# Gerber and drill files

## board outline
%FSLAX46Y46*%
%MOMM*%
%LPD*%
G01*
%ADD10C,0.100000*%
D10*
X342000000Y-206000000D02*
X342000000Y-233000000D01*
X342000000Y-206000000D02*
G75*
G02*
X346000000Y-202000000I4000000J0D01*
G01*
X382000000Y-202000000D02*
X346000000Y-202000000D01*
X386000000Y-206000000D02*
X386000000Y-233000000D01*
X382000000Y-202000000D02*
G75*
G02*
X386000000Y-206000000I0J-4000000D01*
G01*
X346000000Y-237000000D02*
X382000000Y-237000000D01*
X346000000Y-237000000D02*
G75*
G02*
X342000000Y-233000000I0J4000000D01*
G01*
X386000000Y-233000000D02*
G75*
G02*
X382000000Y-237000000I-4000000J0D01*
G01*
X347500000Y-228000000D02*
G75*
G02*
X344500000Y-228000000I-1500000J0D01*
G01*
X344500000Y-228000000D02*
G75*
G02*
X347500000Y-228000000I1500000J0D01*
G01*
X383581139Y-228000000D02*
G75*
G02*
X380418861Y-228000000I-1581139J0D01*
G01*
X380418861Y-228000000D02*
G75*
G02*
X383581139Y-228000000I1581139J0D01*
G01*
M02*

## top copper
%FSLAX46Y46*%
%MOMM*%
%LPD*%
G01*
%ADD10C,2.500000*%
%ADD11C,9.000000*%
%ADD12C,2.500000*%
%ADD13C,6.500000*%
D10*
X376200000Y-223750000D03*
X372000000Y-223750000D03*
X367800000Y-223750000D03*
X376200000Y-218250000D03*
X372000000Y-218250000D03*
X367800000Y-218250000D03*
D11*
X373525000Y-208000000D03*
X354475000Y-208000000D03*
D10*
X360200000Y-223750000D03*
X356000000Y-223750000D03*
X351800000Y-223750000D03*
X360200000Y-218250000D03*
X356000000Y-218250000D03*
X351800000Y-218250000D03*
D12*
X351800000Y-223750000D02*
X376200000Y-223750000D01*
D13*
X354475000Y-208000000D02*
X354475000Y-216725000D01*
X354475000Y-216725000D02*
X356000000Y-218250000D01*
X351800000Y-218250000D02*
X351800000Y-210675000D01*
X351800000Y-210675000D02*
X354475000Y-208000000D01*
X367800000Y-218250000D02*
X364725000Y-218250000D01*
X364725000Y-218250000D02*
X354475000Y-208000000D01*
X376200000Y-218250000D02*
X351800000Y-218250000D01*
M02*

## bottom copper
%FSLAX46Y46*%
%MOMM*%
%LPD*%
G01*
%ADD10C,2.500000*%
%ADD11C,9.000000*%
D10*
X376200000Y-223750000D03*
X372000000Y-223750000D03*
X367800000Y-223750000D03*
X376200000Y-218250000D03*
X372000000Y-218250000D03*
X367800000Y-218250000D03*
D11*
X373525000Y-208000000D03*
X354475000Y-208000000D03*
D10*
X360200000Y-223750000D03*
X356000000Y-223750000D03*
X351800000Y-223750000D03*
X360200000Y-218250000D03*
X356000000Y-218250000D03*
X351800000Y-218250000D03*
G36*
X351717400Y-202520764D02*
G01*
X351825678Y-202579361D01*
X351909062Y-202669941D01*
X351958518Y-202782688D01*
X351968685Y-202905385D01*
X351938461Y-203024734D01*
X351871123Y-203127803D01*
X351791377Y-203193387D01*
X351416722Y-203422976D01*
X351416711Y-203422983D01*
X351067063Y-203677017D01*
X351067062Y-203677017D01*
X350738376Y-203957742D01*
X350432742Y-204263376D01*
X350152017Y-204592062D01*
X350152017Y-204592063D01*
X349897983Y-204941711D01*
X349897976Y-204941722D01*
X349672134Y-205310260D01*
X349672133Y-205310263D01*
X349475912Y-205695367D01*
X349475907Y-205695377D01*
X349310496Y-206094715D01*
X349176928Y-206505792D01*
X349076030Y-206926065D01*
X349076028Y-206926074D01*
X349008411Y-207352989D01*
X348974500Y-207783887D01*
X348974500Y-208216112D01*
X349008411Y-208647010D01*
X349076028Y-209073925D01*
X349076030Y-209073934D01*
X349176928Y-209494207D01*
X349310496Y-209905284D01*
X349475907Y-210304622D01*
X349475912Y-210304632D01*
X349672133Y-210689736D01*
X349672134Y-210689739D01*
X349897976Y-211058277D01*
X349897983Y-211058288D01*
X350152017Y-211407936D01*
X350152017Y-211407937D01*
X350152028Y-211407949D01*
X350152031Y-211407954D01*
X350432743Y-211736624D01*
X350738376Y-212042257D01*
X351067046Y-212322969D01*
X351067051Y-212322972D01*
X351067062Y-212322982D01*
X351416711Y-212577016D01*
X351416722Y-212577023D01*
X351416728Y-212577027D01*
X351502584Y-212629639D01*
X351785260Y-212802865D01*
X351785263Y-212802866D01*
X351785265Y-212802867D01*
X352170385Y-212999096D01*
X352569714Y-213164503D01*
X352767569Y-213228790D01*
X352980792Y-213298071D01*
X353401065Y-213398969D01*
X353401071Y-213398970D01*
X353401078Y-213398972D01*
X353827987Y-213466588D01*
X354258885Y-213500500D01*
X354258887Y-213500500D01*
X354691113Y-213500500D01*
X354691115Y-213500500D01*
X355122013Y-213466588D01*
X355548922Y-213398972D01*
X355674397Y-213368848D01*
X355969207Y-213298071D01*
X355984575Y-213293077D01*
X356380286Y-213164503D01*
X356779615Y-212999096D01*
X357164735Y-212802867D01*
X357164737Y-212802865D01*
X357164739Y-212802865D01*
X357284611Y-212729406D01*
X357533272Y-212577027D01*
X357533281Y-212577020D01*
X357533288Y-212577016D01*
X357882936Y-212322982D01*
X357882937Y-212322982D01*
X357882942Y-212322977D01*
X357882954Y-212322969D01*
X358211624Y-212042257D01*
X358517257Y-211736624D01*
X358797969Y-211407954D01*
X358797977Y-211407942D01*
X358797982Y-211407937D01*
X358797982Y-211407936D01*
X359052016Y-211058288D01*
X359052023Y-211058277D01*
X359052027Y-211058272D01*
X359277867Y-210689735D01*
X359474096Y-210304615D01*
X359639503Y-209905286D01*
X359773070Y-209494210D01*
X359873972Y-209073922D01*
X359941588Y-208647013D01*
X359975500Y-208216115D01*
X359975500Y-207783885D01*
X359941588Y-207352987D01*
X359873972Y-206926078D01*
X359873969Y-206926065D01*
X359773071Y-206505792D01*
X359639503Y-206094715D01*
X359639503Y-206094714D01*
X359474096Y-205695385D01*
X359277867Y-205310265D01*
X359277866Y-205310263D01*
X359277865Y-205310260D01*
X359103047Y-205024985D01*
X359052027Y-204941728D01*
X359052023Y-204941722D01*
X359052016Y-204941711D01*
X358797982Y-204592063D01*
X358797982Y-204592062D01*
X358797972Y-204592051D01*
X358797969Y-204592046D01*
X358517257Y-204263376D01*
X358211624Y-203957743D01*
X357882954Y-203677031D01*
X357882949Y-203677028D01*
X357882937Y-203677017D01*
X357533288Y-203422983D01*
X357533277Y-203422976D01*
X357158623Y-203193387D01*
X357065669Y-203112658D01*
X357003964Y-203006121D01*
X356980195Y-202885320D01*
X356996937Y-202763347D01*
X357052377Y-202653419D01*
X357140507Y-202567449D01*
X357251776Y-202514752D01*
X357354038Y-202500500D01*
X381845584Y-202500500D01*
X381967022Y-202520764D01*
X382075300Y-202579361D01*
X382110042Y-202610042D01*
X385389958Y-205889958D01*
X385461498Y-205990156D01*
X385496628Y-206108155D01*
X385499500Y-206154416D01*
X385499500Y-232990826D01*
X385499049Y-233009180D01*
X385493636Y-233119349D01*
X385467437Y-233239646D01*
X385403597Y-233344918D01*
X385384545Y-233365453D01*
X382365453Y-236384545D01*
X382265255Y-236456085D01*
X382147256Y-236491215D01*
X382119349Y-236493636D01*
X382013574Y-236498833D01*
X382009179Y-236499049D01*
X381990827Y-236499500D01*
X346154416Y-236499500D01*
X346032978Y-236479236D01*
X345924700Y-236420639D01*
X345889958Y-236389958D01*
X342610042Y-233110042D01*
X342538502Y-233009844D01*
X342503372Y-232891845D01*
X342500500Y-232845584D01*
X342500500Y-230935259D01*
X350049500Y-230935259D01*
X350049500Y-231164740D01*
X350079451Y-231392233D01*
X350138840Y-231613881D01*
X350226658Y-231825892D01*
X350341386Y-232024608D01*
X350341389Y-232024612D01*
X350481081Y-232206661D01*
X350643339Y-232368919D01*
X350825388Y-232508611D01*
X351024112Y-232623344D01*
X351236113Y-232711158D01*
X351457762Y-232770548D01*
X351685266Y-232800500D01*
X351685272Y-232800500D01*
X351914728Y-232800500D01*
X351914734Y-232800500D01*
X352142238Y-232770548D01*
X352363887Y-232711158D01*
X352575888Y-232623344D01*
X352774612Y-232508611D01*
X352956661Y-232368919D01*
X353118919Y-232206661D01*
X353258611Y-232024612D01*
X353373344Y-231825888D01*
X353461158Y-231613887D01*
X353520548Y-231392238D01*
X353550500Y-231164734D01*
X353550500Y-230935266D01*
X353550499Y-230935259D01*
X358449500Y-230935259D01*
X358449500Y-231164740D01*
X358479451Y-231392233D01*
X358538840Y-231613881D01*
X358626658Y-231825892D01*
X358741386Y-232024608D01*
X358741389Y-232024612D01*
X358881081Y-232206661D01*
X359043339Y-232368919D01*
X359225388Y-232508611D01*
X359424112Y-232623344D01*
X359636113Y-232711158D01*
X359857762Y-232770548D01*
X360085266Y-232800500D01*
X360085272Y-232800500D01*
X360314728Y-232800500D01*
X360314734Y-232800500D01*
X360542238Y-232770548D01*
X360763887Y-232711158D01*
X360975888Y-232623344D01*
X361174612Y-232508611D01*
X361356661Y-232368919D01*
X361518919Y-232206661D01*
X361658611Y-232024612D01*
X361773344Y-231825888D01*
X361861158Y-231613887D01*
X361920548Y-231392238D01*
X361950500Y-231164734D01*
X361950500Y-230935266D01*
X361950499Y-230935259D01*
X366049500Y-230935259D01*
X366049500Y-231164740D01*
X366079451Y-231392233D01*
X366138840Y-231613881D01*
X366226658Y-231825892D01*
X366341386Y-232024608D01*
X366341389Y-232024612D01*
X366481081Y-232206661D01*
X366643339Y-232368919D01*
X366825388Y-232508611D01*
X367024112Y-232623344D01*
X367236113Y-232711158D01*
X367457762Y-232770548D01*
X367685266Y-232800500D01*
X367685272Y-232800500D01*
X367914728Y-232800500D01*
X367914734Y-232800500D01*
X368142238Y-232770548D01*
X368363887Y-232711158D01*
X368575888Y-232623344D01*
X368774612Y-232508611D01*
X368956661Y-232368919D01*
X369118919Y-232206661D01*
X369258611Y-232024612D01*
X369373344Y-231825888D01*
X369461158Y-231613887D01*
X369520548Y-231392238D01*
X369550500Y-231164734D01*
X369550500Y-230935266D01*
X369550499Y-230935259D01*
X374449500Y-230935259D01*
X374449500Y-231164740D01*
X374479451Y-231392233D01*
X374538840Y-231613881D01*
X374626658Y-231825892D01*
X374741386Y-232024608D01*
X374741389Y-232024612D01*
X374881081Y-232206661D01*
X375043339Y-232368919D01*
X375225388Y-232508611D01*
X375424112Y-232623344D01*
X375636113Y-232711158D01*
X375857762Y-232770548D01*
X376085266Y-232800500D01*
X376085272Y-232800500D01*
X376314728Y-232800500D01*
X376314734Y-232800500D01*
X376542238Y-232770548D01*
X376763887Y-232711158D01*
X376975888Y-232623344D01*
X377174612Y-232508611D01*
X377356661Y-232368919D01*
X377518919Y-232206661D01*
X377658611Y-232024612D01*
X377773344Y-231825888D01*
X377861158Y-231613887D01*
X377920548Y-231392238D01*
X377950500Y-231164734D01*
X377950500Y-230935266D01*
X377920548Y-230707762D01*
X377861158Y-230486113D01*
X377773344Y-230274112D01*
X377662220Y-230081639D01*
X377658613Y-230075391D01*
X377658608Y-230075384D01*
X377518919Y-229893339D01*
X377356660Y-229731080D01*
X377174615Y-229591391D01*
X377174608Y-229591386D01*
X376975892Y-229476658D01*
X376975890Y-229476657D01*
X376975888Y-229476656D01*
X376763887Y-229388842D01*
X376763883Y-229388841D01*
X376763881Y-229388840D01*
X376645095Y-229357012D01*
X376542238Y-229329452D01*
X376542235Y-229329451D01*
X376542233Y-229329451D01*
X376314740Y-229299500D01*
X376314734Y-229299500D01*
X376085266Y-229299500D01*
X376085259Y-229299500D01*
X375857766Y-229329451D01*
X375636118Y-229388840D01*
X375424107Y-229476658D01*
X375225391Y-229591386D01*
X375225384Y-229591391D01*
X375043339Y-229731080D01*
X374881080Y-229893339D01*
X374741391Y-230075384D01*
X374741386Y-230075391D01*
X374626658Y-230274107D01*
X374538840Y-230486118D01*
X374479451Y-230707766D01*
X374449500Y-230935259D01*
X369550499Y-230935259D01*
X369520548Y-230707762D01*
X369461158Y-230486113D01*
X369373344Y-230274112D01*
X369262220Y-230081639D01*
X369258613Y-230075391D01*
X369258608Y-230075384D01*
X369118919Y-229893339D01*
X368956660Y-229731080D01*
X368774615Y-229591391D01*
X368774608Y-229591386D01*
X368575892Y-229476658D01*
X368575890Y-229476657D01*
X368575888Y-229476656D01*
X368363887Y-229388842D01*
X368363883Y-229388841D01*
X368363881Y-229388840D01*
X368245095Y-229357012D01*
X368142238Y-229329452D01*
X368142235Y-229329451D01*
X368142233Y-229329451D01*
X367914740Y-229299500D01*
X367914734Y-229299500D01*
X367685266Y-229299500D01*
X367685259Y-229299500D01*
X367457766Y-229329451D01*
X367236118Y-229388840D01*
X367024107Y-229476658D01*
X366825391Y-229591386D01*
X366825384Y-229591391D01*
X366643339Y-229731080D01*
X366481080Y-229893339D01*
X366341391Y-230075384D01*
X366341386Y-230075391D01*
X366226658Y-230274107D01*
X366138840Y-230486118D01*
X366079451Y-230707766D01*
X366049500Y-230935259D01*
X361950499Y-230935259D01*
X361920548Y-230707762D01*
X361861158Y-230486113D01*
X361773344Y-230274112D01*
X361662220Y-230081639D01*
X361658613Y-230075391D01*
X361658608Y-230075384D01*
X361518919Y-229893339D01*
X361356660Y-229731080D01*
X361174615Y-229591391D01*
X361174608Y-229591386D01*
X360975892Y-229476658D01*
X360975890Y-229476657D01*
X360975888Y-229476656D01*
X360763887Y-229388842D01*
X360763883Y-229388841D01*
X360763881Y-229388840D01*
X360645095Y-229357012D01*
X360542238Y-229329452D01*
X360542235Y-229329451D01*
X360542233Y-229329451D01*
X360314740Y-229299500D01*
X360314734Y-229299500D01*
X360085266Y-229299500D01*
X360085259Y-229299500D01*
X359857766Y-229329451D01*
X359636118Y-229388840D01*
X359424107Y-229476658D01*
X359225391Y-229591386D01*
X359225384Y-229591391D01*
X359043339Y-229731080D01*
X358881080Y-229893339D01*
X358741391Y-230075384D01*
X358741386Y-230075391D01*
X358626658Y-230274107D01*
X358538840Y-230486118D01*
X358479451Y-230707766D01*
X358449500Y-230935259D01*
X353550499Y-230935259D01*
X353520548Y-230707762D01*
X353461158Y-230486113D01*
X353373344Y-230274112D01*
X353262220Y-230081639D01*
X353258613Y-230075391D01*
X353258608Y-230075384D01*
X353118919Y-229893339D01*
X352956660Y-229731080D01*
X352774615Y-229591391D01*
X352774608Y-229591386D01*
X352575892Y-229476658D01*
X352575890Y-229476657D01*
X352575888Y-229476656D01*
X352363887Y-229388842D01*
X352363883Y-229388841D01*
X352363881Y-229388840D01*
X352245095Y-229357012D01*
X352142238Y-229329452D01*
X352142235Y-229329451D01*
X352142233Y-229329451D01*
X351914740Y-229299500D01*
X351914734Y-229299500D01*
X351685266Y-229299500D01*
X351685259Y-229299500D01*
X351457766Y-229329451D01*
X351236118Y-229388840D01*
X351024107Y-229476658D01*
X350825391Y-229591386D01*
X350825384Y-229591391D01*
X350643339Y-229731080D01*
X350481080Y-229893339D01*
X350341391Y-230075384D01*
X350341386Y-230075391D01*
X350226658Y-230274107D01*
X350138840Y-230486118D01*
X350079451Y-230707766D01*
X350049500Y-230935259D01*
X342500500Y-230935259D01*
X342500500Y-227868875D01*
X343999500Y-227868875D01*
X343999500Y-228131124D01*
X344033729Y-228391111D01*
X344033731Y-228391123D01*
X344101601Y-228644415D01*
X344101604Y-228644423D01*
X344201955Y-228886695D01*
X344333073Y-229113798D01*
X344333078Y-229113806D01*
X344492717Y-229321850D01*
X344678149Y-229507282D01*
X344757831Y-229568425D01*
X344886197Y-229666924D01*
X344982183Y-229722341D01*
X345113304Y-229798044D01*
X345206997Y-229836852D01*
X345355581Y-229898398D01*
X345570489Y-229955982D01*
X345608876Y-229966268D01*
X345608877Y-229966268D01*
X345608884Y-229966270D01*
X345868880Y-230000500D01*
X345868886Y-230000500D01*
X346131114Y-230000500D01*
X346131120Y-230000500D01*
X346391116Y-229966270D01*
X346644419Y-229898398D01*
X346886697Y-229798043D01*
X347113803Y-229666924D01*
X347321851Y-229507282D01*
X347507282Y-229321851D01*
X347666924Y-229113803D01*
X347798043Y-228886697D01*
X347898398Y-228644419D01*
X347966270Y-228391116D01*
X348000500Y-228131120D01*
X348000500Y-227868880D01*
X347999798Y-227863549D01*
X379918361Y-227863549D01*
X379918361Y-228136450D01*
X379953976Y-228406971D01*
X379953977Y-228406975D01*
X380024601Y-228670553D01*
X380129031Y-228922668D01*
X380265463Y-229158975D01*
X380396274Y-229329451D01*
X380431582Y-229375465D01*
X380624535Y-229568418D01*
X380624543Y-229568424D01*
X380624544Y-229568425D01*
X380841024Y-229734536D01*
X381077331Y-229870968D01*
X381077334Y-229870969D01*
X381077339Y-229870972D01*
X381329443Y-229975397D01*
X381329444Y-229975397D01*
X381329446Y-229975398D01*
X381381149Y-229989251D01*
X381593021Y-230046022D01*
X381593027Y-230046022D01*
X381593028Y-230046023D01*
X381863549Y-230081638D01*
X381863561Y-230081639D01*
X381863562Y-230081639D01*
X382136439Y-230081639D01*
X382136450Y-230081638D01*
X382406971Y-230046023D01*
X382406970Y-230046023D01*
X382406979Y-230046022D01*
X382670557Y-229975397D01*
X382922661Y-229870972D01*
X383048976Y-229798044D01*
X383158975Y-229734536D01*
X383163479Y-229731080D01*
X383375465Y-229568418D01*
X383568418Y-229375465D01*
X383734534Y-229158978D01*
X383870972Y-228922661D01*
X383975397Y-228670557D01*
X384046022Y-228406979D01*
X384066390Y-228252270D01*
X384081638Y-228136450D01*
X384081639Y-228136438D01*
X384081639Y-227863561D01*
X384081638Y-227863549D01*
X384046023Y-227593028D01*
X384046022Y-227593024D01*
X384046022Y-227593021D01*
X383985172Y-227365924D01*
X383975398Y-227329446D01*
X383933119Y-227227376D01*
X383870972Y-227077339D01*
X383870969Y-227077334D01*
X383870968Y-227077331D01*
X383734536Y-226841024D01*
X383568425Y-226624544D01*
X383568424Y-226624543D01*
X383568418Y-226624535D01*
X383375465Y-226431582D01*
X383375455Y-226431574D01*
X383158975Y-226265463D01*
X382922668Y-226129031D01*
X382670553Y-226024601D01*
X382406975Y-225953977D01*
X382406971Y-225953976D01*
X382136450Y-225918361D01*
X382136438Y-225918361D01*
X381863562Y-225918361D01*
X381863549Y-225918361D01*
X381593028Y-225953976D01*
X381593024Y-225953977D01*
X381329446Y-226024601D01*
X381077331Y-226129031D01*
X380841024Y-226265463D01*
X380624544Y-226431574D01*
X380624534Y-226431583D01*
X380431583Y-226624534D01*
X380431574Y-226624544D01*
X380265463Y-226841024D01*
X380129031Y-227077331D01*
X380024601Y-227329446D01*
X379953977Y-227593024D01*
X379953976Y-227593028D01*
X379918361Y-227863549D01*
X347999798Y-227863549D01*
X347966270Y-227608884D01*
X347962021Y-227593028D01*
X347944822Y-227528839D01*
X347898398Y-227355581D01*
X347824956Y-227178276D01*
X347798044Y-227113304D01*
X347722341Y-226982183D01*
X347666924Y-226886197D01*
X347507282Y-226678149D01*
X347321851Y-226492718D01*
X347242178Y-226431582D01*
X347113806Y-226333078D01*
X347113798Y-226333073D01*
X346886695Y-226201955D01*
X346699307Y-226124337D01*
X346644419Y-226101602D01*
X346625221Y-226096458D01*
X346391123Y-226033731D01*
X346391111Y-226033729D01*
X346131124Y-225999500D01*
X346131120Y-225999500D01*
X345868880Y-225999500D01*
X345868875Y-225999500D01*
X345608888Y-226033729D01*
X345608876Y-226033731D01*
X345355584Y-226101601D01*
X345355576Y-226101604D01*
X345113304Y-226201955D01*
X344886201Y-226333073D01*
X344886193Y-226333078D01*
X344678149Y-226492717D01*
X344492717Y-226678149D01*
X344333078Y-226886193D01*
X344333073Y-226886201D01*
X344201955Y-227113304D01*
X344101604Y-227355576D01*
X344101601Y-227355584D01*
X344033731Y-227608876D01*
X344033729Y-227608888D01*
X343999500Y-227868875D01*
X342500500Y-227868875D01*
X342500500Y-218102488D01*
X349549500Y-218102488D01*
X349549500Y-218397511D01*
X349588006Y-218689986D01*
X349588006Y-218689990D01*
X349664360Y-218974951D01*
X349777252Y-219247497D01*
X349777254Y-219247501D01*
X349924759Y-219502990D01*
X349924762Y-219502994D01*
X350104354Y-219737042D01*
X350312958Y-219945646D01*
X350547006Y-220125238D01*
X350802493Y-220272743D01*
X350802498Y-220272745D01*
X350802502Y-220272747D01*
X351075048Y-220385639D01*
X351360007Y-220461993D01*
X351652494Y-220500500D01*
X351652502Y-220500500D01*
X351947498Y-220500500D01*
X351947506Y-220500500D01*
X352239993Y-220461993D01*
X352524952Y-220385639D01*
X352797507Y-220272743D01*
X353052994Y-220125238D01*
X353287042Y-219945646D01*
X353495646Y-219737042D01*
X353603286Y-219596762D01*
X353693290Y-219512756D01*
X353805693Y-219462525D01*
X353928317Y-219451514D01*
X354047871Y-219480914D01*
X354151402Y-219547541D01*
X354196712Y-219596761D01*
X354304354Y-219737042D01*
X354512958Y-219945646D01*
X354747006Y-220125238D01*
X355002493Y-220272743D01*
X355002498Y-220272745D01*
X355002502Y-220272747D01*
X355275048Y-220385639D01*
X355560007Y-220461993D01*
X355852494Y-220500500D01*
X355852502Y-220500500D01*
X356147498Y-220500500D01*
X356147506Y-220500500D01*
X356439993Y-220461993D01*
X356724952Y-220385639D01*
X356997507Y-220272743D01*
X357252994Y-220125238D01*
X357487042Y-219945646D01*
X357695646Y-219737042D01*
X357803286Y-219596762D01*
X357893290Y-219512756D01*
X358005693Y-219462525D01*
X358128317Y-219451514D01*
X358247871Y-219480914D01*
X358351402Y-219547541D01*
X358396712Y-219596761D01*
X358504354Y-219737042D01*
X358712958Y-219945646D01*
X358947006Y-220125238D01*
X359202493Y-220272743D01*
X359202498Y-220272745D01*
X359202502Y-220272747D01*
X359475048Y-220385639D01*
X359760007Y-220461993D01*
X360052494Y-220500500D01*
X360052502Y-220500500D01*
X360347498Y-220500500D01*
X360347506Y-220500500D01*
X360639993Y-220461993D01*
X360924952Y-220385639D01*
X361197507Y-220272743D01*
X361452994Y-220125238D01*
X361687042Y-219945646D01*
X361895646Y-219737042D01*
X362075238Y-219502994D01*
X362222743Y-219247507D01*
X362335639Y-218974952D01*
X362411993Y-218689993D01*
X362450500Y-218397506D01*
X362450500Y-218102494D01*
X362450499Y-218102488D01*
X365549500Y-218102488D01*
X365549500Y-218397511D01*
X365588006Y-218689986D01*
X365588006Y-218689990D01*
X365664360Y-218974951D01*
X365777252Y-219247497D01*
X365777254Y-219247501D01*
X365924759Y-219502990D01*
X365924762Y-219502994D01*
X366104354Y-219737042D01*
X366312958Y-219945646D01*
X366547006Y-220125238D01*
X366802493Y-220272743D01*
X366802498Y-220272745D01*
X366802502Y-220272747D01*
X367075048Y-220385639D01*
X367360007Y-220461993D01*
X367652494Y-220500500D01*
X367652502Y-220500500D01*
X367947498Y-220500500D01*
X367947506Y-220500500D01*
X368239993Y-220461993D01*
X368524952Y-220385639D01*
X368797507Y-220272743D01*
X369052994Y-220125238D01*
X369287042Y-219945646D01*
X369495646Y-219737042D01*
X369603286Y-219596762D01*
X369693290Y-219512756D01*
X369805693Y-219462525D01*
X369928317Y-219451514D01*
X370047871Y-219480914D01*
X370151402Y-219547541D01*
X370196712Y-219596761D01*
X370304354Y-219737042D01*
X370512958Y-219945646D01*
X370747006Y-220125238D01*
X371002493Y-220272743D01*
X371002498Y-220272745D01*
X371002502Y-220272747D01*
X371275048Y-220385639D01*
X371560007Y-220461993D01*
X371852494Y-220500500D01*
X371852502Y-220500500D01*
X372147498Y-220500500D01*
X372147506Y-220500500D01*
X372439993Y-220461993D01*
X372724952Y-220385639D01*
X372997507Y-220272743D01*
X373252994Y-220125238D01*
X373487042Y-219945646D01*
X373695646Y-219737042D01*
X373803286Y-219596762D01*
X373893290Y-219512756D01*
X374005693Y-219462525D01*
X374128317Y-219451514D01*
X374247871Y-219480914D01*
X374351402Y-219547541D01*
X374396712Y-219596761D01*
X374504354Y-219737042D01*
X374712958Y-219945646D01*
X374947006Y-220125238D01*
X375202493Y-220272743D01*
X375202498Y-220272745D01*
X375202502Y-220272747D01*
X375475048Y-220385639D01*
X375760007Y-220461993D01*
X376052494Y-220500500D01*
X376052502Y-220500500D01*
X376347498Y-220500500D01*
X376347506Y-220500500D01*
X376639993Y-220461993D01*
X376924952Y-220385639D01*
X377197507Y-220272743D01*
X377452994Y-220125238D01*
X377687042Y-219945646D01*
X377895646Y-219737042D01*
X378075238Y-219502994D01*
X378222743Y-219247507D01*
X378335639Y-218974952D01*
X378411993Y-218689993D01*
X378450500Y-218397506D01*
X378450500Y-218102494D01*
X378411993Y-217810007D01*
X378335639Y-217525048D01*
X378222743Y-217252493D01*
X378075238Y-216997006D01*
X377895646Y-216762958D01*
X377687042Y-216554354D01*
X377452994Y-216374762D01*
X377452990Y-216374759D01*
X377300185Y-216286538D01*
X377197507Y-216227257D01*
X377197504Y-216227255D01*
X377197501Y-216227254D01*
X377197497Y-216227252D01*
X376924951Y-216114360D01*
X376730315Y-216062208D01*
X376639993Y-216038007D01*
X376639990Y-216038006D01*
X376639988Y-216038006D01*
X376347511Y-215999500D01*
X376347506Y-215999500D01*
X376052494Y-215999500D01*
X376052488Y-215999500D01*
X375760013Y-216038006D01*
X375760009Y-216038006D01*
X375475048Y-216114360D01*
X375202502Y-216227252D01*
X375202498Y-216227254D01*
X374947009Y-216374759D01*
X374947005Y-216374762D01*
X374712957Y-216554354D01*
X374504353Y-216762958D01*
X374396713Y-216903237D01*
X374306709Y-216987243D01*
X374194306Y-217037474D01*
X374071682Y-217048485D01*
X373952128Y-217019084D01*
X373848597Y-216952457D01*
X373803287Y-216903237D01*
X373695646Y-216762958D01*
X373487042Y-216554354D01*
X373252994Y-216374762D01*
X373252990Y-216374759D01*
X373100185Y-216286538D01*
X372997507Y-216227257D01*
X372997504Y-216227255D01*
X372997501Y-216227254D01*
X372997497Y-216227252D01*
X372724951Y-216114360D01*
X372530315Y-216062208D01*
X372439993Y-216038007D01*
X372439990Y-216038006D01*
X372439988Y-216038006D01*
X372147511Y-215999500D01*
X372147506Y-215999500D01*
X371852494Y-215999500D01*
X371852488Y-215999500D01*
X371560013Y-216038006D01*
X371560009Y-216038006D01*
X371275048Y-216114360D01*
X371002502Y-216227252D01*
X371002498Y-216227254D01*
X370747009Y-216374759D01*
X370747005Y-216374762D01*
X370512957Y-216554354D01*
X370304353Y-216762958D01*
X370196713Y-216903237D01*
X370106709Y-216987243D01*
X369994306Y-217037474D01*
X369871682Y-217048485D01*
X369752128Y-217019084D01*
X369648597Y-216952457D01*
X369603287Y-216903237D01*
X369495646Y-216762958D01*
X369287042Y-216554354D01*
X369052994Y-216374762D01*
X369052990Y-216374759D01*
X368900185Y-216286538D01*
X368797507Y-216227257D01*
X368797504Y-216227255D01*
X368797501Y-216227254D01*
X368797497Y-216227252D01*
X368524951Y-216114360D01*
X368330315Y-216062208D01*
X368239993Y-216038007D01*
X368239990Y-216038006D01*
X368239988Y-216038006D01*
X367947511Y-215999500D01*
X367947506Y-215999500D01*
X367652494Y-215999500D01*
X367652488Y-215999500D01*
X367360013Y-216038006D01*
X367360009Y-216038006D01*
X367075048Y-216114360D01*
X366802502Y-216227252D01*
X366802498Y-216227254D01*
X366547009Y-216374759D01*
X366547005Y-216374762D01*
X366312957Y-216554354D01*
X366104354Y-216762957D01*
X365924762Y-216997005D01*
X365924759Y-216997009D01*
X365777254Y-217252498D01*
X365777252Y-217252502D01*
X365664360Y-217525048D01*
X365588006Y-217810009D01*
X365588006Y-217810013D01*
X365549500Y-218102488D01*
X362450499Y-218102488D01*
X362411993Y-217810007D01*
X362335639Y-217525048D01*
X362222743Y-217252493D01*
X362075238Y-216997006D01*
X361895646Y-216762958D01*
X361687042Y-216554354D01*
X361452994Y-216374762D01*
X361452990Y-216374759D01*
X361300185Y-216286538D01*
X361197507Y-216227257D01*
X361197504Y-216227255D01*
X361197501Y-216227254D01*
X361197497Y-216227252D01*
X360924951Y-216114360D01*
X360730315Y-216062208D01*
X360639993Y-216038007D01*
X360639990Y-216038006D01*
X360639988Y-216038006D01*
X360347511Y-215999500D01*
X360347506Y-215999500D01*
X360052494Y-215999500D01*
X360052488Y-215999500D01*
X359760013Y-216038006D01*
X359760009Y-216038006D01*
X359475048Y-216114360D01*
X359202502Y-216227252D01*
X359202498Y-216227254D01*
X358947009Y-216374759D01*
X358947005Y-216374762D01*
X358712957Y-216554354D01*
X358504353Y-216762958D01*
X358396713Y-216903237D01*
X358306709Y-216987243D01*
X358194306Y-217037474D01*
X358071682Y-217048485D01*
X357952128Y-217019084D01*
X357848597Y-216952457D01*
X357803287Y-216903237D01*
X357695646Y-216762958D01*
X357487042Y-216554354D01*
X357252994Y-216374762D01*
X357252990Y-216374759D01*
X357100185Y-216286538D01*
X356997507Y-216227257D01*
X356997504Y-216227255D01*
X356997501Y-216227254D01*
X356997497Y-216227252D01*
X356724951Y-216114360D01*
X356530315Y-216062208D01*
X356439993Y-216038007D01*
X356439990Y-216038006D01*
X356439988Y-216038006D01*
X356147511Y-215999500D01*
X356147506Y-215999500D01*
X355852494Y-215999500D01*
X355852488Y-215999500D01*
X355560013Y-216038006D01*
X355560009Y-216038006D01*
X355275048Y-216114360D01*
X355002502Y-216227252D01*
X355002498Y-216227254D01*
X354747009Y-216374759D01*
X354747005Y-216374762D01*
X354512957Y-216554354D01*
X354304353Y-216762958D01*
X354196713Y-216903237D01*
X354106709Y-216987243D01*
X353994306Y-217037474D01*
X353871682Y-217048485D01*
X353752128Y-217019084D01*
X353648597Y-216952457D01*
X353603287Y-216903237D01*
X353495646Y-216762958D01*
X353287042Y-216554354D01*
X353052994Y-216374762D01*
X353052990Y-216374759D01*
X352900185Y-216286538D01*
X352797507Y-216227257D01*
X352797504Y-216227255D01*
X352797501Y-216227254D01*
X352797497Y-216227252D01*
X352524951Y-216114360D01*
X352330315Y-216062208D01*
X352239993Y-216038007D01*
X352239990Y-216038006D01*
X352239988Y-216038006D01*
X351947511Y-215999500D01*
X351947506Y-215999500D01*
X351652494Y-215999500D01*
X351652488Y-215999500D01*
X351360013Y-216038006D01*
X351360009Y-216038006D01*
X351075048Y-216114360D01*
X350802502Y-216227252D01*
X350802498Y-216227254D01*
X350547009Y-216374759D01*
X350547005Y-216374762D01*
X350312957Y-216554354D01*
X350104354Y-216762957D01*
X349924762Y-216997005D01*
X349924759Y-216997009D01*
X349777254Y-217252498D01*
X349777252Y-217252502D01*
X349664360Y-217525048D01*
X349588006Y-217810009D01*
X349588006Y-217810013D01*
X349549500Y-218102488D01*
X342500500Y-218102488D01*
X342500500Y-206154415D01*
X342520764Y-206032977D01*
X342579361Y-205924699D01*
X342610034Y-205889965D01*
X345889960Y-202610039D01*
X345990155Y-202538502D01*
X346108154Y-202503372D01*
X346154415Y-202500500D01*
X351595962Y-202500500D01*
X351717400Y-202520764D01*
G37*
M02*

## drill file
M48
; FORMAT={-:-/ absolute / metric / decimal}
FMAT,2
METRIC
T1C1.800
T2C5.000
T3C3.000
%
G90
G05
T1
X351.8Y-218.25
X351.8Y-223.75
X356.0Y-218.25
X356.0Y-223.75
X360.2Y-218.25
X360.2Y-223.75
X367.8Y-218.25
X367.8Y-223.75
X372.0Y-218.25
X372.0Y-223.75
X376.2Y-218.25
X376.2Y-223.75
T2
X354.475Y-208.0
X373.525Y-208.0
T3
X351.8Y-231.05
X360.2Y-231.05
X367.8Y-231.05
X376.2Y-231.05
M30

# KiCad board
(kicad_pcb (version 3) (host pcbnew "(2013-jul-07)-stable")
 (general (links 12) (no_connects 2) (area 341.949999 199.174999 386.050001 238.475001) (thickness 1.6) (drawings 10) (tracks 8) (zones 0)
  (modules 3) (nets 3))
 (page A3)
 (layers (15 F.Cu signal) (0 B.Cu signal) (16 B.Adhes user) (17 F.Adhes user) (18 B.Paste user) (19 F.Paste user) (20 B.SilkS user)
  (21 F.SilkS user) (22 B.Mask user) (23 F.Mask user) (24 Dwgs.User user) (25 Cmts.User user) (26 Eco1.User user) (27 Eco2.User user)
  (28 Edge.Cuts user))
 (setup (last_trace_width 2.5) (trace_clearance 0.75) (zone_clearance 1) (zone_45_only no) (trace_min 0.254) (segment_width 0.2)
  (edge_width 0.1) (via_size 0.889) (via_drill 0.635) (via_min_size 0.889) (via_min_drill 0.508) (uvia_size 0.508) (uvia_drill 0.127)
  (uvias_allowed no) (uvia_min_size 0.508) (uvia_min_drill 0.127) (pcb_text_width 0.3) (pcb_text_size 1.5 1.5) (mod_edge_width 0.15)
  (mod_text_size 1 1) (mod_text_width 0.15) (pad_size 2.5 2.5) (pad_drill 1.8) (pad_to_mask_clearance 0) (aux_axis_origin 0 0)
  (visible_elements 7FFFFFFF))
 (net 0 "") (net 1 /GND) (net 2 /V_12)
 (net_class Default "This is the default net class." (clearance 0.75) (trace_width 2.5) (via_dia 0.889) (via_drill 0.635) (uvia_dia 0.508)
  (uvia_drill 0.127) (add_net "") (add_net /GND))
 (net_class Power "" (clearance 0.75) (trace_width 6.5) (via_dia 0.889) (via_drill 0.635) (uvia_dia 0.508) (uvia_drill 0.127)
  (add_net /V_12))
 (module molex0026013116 (layer F.Cu) (at 372 221)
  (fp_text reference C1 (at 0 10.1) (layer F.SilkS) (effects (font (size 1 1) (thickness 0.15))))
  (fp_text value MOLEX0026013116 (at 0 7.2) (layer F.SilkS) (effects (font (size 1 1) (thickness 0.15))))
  (pad 1 thru_hole circle (at 4.2 2.75) (size 2.5 2.5) (drill 1.8) (layers *.Cu *.Mask F.SilkS) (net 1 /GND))
  (pad 2 thru_hole circle (at 0 2.75) (size 2.5 2.5) (drill 1.8) (layers *.Cu *.Mask F.SilkS) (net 1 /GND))
  (pad 3 thru_hole circle (at -4.2 2.75) (size 2.5 2.5) (drill 1.8) (layers *.Cu *.Mask F.SilkS) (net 1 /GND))
  (pad 4 thru_hole circle (at 4.2 -2.75) (size 2.5 2.5) (drill 1.8) (layers *.Cu *.Mask F.SilkS) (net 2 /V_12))
  (pad 5 thru_hole circle (at 0 -2.75) (size 2.5 2.5) (drill 1.8) (layers *.Cu *.Mask F.SilkS) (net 2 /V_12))
  (pad 6 thru_hole circle (at -4.2 -2.75) (size 2.5 2.5) (drill 1.8) (layers *.Cu *.Mask F.SilkS) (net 2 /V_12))
  (pad "" np_thru_hole circle (at 4.2 10.05) (size 3 3) (drill 3) (layers *.Cu *.Mask F.SilkS))
  (pad "" np_thru_hole circle (at -4.2 10.05) (size 3 3) (drill 3) (layers *.Cu *.Mask F.SilkS)))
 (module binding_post (layer F.Cu) (at 364 208)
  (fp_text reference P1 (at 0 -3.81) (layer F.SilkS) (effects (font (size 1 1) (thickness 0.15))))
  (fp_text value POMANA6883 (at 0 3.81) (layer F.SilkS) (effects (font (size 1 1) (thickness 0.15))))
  (pad 1 thru_hole circle (at 9.525 0) (size 9 9) (drill 5) (layers *.Cu *.Mask F.SilkS) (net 1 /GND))
  (pad 2 thru_hole circle (at -9.525 0) (size 9 9) (drill 5) (layers *.Cu *.Mask F.SilkS) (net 2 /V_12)))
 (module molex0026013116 (layer F.Cu) (at 356 221)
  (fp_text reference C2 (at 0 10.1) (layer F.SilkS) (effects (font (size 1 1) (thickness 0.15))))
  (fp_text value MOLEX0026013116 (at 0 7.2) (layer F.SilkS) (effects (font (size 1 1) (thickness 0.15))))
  (pad 1 thru_hole circle (at 4.2 2.75) (size 2.5 2.5) (drill 1.8) (layers *.Cu *.Mask F.SilkS) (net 1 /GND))
  (pad 2 thru_hole circle (at 0 2.75) (size 2.5 2.5) (drill 1.8) (layers *.Cu *.Mask F.SilkS) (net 1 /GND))
  (pad 3 thru_hole circle (at -4.2 2.75) (size 2.5 2.5) (drill 1.8) (layers *.Cu *.Mask F.SilkS) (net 1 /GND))
  (pad 4 thru_hole circle (at 4.2 -2.75) (size 2.5 2.5) (drill 1.8) (layers *.Cu *.Mask F.SilkS) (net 2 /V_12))
  (pad 5 thru_hole circle (at 0 -2.75) (size 2.5 2.5) (drill 1.8) (layers *.Cu *.Mask F.SilkS) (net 2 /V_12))
  (pad 6 thru_hole circle (at -4.2 -2.75) (size 2.5 2.5) (drill 1.8) (layers *.Cu *.Mask F.SilkS) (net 2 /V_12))
  (pad "" np_thru_hole circle (at 4.2 10.05) (size 3 3) (drill 3) (layers *.Cu *.Mask F.SilkS))
  (pad "" np_thru_hole circle (at -4.2 10.05) (size 3 3) (drill 3) (layers *.Cu *.Mask F.SilkS)))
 (gr_line (start 342 206) (end 342 233) (angle 90) (layer Edge.Cuts) (width 0.1))
 (gr_arc (start 346 206) (end 342 206) (angle 90) (layer Edge.Cuts) (width 0.1))
 (gr_line (start 382 202) (end 346 202) (angle 90) (layer Edge.Cuts) (width 0.1))
 (gr_line (start 386 206) (end 386 233) (angle 90) (layer Edge.Cuts) (width 0.1))
 (gr_arc (start 382 206) (end 382 202) (angle 90) (layer Edge.Cuts) (width 0.1))
 (gr_line (start 346 237) (end 382 237) (angle 90) (layer Edge.Cuts) (width 0.1))
 (gr_arc (start 346 233) (end 346 237) (angle 90) (layer Edge.Cuts) (width 0.1))
 (gr_arc (start 382 233) (end 386 233) (angle 90) (layer Edge.Cuts) (width 0.1))
 (gr_circle (center 346 228) (end 347.5 228) (layer Edge.Cuts) (width 0.1))
 (gr_circle (center 382 228) (end 380.5 227.5) (layer Edge.Cuts) (width 0.1))
 (segment (start 351.8 223.75) (end 376.2 223.75) (width 2.5) (layer F.Cu) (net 1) (status C00000))
 (segment (start 354.475 208) (end 354.475 216.725) (width 6.5) (layer F.Cu) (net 2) (status 400000))
 (segment (start 354.475 216.725) (end 356 218.25) (width 6.5) (layer F.Cu) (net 2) (status 800000))
 (segment (start 351.8 218.25) (end 351.8 210.675) (width 6.5) (layer F.Cu) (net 2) (status C00000))
 (segment (start 351.8 210.675) (end 354.475 208) (width 6.5) (layer F.Cu) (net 2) (status C00000))
 (segment (start 367.8 218.25) (end 364.725 218.25) (width 6.5) (layer F.Cu) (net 2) (status 400000))
 (segment (start 364.725 218.25) (end 354.475 208) (width 6.5) (layer F.Cu) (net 2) (status 800000))
 (segment (start 376.2 218.25) (end 351.8 218.25) (width 6.5) (layer F.Cu) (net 2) (status C00000))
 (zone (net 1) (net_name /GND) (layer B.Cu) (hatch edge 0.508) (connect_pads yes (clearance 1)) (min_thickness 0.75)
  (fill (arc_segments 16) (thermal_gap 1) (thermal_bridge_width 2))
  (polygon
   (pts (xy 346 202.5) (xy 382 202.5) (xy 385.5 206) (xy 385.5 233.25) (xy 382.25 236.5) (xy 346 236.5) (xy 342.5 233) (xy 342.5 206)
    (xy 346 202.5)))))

